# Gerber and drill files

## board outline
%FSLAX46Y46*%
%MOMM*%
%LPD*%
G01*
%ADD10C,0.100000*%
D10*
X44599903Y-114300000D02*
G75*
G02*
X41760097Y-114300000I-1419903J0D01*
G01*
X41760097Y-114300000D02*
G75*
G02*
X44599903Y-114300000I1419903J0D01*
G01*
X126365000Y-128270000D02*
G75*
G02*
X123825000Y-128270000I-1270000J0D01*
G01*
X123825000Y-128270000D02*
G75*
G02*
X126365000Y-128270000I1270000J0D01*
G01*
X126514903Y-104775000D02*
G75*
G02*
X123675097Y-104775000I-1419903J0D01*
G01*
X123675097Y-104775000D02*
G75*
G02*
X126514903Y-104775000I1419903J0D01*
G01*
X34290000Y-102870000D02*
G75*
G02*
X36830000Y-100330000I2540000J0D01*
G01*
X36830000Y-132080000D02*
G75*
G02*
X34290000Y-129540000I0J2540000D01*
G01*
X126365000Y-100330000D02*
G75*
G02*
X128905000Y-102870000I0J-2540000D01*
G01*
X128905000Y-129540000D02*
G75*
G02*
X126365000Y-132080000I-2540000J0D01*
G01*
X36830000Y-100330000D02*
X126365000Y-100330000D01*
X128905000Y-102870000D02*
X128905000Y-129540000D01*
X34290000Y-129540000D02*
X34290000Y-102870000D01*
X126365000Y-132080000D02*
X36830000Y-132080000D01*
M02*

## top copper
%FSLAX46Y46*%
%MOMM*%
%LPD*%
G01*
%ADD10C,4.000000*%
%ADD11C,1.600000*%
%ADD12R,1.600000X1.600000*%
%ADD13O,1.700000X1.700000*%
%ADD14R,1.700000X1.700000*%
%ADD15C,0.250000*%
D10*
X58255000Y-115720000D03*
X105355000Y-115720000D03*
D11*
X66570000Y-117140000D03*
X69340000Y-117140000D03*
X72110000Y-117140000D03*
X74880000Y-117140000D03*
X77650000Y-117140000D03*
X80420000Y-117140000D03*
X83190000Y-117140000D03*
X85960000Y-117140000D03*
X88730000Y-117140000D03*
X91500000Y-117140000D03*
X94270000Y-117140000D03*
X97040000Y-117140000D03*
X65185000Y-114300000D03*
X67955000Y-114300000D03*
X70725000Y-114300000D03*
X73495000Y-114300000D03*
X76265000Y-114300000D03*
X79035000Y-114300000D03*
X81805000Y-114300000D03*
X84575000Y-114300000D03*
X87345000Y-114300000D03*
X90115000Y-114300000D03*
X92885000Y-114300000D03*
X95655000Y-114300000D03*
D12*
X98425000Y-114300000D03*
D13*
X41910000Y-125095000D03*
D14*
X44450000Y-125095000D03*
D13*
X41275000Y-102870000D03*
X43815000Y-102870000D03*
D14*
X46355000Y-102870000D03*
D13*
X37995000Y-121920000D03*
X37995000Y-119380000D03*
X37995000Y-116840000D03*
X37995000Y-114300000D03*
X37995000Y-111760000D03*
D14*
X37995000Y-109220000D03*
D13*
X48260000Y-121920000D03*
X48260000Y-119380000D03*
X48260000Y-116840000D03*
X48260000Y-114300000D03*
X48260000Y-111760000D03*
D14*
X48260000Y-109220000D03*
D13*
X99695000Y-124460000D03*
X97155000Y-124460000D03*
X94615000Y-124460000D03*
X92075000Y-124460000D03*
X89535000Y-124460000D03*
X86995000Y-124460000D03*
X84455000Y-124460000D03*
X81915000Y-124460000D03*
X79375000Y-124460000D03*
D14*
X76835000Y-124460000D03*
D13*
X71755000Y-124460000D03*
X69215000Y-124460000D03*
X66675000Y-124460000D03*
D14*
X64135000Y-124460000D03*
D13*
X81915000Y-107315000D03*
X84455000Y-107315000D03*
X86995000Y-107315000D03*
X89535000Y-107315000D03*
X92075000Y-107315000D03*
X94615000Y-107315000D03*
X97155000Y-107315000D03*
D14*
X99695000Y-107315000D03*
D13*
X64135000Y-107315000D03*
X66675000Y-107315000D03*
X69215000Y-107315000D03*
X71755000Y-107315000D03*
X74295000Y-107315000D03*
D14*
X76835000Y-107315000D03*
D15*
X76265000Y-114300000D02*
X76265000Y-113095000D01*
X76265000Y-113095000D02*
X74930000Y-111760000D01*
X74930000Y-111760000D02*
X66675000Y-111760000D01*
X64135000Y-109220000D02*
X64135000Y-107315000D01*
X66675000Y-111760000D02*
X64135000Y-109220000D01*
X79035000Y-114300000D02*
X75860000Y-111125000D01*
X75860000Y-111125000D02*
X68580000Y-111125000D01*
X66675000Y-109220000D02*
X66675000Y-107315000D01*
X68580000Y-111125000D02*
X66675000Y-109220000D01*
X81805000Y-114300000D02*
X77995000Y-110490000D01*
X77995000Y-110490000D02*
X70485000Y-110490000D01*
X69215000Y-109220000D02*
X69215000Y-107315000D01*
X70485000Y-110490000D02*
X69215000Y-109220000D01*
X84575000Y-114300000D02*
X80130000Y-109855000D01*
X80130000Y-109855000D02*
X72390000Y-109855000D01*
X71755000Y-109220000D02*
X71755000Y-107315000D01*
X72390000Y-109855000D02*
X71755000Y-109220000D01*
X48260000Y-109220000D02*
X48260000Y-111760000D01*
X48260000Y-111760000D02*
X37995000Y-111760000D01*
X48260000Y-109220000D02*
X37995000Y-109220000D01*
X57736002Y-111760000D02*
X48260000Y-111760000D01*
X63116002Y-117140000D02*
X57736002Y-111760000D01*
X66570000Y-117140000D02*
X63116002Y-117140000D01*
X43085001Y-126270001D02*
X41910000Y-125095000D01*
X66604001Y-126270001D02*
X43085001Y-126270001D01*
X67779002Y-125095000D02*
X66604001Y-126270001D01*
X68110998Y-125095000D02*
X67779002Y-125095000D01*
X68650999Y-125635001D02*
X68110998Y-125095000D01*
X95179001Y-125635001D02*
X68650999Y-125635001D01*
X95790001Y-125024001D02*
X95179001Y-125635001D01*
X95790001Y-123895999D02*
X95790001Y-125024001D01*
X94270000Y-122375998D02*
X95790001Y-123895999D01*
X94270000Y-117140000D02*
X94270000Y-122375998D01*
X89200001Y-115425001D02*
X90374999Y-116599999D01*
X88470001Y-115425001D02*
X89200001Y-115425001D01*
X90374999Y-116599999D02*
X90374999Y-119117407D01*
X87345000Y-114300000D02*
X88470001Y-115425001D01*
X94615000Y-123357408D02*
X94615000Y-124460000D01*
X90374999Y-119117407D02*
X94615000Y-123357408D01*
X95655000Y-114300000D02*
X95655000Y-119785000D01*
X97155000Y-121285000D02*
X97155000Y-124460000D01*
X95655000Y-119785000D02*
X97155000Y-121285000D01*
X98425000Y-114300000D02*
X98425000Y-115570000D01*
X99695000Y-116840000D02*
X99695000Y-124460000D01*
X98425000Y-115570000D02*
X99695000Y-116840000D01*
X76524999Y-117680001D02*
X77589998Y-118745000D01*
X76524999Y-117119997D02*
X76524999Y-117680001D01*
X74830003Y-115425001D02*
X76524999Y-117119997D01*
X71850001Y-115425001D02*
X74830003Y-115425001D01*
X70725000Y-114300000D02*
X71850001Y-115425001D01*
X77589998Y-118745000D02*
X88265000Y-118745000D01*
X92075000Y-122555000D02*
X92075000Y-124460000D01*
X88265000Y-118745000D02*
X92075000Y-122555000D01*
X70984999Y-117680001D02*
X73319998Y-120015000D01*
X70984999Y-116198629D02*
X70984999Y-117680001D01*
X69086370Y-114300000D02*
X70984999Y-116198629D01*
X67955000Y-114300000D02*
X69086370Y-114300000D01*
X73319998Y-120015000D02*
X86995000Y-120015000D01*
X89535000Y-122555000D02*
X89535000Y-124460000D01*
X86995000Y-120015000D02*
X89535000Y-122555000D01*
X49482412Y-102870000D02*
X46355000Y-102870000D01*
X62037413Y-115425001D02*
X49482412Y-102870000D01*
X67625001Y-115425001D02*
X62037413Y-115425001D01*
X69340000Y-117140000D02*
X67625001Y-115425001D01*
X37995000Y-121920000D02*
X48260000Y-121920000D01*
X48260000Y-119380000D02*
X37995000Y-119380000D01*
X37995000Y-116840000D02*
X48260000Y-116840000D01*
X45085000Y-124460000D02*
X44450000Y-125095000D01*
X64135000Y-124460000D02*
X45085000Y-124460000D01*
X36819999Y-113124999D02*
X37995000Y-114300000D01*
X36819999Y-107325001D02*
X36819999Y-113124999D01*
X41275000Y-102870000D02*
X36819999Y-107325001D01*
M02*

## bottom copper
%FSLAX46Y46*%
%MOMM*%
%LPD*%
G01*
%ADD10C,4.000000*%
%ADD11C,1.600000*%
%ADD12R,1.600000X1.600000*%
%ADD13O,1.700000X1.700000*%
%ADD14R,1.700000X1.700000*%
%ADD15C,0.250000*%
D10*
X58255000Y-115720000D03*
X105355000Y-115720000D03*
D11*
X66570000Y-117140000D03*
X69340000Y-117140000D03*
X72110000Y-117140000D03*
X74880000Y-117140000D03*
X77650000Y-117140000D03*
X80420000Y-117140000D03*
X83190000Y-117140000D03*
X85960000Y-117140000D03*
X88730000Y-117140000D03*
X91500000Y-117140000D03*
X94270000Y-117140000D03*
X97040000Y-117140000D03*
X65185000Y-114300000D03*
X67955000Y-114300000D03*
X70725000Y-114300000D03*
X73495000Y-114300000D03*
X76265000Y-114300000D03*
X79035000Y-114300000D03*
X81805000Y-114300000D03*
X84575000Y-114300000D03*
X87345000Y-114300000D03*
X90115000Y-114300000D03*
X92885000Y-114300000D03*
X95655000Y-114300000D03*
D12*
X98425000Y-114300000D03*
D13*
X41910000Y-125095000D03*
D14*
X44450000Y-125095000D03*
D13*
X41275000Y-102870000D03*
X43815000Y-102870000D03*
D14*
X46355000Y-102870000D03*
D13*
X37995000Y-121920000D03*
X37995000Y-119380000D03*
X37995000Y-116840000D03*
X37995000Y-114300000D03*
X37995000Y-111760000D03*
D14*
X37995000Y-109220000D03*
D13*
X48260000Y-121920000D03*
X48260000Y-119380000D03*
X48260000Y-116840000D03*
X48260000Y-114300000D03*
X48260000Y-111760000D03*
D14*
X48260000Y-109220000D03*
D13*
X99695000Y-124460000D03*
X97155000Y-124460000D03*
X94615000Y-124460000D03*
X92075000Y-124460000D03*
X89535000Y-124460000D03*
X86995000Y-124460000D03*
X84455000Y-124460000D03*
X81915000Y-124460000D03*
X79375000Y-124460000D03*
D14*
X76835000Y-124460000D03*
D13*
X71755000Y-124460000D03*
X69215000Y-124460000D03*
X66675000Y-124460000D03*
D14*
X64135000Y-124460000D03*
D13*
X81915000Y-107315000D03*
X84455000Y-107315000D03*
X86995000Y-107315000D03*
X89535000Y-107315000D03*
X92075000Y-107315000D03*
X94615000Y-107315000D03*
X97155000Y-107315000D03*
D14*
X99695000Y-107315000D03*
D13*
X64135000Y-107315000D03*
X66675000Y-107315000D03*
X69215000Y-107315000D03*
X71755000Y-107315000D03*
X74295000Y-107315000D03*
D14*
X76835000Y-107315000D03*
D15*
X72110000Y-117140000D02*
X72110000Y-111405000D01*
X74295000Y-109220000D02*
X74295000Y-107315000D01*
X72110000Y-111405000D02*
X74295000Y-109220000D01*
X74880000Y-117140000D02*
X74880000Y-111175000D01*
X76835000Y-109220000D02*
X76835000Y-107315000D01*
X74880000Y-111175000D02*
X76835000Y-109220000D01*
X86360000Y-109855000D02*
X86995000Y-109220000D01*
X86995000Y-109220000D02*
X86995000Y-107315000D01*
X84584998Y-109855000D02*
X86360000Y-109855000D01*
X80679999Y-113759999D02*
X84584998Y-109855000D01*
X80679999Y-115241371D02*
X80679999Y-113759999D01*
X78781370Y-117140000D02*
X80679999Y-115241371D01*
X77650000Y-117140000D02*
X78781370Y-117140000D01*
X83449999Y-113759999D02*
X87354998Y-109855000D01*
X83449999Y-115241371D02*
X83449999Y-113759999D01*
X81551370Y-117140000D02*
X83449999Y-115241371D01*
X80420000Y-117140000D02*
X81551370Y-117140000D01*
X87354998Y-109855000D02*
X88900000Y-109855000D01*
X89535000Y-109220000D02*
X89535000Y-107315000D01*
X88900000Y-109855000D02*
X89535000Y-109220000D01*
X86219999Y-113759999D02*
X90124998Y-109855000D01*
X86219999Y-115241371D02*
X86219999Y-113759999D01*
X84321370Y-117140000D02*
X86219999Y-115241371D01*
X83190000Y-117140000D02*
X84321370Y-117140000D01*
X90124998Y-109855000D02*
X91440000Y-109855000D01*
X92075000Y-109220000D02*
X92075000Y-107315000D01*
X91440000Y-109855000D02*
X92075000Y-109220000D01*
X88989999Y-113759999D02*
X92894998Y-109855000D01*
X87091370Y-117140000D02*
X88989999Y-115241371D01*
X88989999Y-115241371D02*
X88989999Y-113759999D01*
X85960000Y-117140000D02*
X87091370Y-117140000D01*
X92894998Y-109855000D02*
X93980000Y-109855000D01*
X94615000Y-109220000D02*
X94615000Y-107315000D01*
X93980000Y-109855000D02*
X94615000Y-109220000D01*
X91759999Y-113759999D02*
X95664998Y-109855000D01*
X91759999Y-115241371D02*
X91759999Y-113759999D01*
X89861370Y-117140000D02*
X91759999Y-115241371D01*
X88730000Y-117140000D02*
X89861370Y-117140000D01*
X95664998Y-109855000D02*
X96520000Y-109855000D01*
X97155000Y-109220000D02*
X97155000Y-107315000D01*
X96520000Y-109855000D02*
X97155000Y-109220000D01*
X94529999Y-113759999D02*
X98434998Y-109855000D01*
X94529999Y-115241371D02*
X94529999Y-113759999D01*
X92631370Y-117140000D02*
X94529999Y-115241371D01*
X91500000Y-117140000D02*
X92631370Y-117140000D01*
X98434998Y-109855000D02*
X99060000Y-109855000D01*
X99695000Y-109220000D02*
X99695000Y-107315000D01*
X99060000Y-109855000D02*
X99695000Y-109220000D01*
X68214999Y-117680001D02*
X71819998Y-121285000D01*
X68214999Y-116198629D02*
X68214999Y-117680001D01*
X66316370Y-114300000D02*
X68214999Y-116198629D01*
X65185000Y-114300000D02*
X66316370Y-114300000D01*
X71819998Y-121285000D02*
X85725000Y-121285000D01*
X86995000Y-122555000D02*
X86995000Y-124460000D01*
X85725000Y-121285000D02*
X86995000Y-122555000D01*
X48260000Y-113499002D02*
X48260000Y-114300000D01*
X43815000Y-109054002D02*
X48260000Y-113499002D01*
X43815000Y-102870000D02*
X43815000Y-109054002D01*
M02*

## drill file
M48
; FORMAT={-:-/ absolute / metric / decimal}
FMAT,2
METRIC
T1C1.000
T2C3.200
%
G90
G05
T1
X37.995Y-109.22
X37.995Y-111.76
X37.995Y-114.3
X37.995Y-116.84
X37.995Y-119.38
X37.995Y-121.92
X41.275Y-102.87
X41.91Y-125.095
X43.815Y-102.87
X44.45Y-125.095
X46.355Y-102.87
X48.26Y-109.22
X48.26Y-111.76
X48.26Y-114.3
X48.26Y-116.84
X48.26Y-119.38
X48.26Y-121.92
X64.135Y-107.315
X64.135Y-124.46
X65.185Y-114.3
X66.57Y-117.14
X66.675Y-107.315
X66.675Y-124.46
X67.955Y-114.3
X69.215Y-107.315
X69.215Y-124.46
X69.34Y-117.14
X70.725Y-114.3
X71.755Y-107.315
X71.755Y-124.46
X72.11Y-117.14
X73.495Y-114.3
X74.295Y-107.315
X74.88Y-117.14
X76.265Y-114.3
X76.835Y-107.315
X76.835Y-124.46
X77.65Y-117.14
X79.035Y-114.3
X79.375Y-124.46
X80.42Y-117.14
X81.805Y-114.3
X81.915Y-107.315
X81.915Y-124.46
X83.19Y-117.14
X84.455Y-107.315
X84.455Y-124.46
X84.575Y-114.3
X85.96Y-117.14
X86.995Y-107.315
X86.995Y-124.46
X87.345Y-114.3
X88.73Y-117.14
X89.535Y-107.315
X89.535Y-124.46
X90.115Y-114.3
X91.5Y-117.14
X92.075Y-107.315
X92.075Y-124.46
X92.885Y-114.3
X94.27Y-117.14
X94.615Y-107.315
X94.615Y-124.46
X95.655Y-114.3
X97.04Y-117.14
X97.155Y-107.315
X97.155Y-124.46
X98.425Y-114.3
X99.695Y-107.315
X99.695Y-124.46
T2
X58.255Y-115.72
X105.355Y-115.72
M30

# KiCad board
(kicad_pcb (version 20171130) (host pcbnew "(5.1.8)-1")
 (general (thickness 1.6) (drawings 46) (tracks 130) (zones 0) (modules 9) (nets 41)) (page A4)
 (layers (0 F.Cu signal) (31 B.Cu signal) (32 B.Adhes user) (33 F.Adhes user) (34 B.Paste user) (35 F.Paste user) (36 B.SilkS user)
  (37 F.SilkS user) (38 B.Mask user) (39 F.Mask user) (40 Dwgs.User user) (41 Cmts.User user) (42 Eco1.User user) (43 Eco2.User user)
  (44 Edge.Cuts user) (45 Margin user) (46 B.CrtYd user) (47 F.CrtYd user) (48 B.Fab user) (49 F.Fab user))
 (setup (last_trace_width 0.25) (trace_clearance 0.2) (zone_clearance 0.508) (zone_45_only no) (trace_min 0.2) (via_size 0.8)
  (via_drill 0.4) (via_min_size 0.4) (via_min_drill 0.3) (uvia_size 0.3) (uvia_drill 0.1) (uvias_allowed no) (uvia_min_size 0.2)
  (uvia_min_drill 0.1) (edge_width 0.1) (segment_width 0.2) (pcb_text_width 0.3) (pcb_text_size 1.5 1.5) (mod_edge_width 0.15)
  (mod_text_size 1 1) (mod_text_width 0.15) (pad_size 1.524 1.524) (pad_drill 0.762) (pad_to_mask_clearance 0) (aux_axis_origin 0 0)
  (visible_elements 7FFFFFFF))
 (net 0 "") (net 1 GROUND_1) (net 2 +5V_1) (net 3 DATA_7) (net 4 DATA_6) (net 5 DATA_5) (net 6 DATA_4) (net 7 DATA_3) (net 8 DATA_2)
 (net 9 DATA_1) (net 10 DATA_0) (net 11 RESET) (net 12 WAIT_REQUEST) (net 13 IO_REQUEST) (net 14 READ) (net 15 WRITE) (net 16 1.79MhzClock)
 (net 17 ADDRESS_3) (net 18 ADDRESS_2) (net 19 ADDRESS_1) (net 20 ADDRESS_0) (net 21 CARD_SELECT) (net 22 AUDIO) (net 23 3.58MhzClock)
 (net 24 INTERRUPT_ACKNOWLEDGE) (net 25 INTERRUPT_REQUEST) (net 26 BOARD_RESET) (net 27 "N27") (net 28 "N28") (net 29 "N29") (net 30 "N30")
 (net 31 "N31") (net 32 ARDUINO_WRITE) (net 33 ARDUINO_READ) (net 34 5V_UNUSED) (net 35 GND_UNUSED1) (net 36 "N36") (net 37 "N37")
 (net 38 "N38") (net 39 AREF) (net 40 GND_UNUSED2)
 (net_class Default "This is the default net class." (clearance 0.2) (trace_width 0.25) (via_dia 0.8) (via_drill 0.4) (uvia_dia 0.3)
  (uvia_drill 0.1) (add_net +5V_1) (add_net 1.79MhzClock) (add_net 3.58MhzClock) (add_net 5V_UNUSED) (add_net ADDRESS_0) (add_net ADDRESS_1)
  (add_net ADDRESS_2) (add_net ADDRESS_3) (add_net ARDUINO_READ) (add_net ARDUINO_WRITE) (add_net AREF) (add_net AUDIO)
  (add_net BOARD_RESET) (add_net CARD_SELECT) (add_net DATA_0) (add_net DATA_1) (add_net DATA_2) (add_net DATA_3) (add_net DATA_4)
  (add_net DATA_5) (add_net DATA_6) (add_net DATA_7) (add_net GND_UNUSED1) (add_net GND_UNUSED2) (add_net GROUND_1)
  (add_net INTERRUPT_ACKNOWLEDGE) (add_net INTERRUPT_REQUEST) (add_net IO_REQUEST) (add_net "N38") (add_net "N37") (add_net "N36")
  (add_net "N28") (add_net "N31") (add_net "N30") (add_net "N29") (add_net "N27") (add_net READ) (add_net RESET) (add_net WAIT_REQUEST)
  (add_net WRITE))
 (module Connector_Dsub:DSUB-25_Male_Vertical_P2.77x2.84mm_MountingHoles (layer B.Cu) (at 98.425 114.3 180)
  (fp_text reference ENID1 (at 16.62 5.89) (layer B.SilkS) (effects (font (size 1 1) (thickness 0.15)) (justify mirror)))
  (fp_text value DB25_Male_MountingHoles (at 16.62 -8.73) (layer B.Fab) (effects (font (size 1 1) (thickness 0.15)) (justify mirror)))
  (pad 0 thru_hole circle (at 40.17 -1.42 180) (size 4 4) (drill 3.2) (layers *.Cu *.Mask))
  (pad 0 thru_hole circle (at -6.93 -1.42 180) (size 4 4) (drill 3.2) (layers *.Cu *.Mask))
  (pad 25 thru_hole circle (at 31.855 -2.84 180) (size 1.6 1.6) (drill 1) (layers *.Cu *.Mask) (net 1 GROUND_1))
  (pad 24 thru_hole circle (at 29.085 -2.84 180) (size 1.6 1.6) (drill 1) (layers *.Cu *.Mask) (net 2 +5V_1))
  (pad 23 thru_hole circle (at 26.315 -2.84 180) (size 1.6 1.6) (drill 1) (layers *.Cu *.Mask) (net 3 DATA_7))
  (pad 22 thru_hole circle (at 23.545 -2.84 180) (size 1.6 1.6) (drill 1) (layers *.Cu *.Mask) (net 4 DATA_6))
  (pad 21 thru_hole circle (at 20.775 -2.84 180) (size 1.6 1.6) (drill 1) (layers *.Cu *.Mask) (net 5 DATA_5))
  (pad 20 thru_hole circle (at 18.005 -2.84 180) (size 1.6 1.6) (drill 1) (layers *.Cu *.Mask) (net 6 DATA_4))
  (pad 19 thru_hole circle (at 15.235 -2.84 180) (size 1.6 1.6) (drill 1) (layers *.Cu *.Mask) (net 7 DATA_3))
  (pad 18 thru_hole circle (at 12.465 -2.84 180) (size 1.6 1.6) (drill 1) (layers *.Cu *.Mask) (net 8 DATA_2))
  (pad 17 thru_hole circle (at 9.695 -2.84 180) (size 1.6 1.6) (drill 1) (layers *.Cu *.Mask) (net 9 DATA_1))
  (pad 16 thru_hole circle (at 6.925 -2.84 180) (size 1.6 1.6) (drill 1) (layers *.Cu *.Mask) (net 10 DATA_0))
  (pad 15 thru_hole circle (at 4.155 -2.84 180) (size 1.6 1.6) (drill 1) (layers *.Cu *.Mask) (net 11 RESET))
  (pad 14 thru_hole circle (at 1.385 -2.84 180) (size 1.6 1.6) (drill 1) (layers *.Cu *.Mask) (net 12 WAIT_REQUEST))
  (pad 13 thru_hole circle (at 33.24 0 180) (size 1.6 1.6) (drill 1) (layers *.Cu *.Mask) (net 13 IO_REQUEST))
  (pad 12 thru_hole circle (at 30.47 0 180) (size 1.6 1.6) (drill 1) (layers *.Cu *.Mask) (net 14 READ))
  (pad 11 thru_hole circle (at 27.7 0 180) (size 1.6 1.6) (drill 1) (layers *.Cu *.Mask) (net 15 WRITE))
  (pad 10 thru_hole circle (at 24.93 0 180) (size 1.6 1.6) (drill 1) (layers *.Cu *.Mask) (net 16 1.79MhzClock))
  (pad 9 thru_hole circle (at 22.16 0 180) (size 1.6 1.6) (drill 1) (layers *.Cu *.Mask) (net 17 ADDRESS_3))
  (pad 8 thru_hole circle (at 19.39 0 180) (size 1.6 1.6) (drill 1) (layers *.Cu *.Mask) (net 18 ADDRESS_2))
  (pad 7 thru_hole circle (at 16.62 0 180) (size 1.6 1.6) (drill 1) (layers *.Cu *.Mask) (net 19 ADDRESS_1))
  (pad 6 thru_hole circle (at 13.85 0 180) (size 1.6 1.6) (drill 1) (layers *.Cu *.Mask) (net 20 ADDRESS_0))
  (pad 5 thru_hole circle (at 11.08 0 180) (size 1.6 1.6) (drill 1) (layers *.Cu *.Mask) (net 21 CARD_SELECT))
  (pad 4 thru_hole circle (at 8.31 0 180) (size 1.6 1.6) (drill 1) (layers *.Cu *.Mask) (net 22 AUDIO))
  (pad 3 thru_hole circle (at 5.54 0 180) (size 1.6 1.6) (drill 1) (layers *.Cu *.Mask) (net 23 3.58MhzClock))
  (pad 2 thru_hole circle (at 2.77 0 180) (size 1.6 1.6) (drill 1) (layers *.Cu *.Mask) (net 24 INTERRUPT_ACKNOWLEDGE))
  (pad 1 thru_hole rect (at 0 0 180) (size 1.6 1.6) (drill 1) (layers *.Cu *.Mask) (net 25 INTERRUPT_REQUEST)))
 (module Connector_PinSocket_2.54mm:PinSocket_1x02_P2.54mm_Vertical (layer F.Cu) (at 44.45 125.095 270)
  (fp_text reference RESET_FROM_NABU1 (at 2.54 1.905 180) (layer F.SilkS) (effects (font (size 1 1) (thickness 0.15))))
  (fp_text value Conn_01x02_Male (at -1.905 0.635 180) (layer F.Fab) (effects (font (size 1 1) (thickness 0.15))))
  (pad 2 thru_hole oval (at 0 2.54 270) (size 1.7 1.7) (drill 1) (layers *.Cu *.Mask) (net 11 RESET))
  (pad 1 thru_hole rect (at 0 0 270) (size 1.7 1.7) (drill 1) (layers *.Cu *.Mask) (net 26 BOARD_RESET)))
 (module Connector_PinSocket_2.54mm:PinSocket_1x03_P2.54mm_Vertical (layer F.Cu) (at 46.355 102.87 270)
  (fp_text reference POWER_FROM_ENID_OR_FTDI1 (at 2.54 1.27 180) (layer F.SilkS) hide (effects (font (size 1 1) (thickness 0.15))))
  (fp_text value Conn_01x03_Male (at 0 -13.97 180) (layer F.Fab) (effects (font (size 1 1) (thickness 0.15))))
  (pad 3 thru_hole oval (at 0 5.08 270) (size 1.7 1.7) (drill 1) (layers *.Cu *.Mask) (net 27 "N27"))
  (pad 2 thru_hole oval (at 0 2.54 270) (size 1.7 1.7) (drill 1) (layers *.Cu *.Mask) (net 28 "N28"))
  (pad 1 thru_hole rect (at 0 0 270) (size 1.7 1.7) (drill 1) (layers *.Cu *.Mask) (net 2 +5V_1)))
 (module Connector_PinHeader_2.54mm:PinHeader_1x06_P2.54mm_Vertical (layer F.Cu) (at 37.995 109.22)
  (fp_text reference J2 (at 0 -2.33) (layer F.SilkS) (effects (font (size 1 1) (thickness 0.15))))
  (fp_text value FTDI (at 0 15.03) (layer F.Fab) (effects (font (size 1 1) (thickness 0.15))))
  (pad 6 thru_hole oval (at 0 12.7) (size 1.7 1.7) (drill 1) (layers *.Cu *.Mask) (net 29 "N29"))
  (pad 5 thru_hole oval (at 0 10.16) (size 1.7 1.7) (drill 1) (layers *.Cu *.Mask) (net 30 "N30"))
  (pad 4 thru_hole oval (at 0 7.62) (size 1.7 1.7) (drill 1) (layers *.Cu *.Mask) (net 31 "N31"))
  (pad 3 thru_hole oval (at 0 5.08) (size 1.7 1.7) (drill 1) (layers *.Cu *.Mask) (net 27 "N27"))
  (pad 2 thru_hole oval (at 0 2.54) (size 1.7 1.7) (drill 1) (layers *.Cu *.Mask) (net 1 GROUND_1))
  (pad 1 thru_hole rect (at 0 0) (size 1.7 1.7) (drill 1) (layers *.Cu *.Mask) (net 1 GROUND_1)))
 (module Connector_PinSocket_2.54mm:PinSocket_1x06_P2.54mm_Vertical (layer F.Cu) (at 48.26 109.22)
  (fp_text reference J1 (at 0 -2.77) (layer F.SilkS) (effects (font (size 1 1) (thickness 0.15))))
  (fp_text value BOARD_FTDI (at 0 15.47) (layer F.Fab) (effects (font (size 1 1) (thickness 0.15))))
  (pad 6 thru_hole oval (at 0 12.7) (size 1.7 1.7) (drill 1) (layers *.Cu *.Mask) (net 29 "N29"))
  (pad 5 thru_hole oval (at 0 10.16) (size 1.7 1.7) (drill 1) (layers *.Cu *.Mask) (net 30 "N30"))
  (pad 4 thru_hole oval (at 0 7.62) (size 1.7 1.7) (drill 1) (layers *.Cu *.Mask) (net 31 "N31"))
  (pad 3 thru_hole oval (at 0 5.08) (size 1.7 1.7) (drill 1) (layers *.Cu *.Mask) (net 28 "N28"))
  (pad 2 thru_hole oval (at 0 2.54) (size 1.7 1.7) (drill 1) (layers *.Cu *.Mask) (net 1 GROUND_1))
  (pad 1 thru_hole rect (at 0 0) (size 1.7 1.7) (drill 1) (layers *.Cu *.Mask) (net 1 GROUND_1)))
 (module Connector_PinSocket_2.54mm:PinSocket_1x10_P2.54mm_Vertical (layer F.Cu) (at 76.835 124.46 90)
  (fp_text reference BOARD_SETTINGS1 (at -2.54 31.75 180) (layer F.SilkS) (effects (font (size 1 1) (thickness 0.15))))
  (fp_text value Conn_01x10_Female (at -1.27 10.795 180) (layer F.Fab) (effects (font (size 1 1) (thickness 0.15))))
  (pad 10 thru_hole oval (at 0 22.86 90) (size 1.7 1.7) (drill 1) (layers *.Cu *.Mask) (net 25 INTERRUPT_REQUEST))
  (pad 9 thru_hole oval (at 0 20.32 90) (size 1.7 1.7) (drill 1) (layers *.Cu *.Mask) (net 24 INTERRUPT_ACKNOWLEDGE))
  (pad 8 thru_hole oval (at 0 17.78 90) (size 1.7 1.7) (drill 1) (layers *.Cu *.Mask) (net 21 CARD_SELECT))
  (pad 7 thru_hole oval (at 0 15.24 90) (size 1.7 1.7) (drill 1) (layers *.Cu *.Mask) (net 15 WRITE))
  (pad 6 thru_hole oval (at 0 12.7 90) (size 1.7 1.7) (drill 1) (layers *.Cu *.Mask) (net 14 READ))
  (pad 5 thru_hole oval (at 0 10.16 90) (size 1.7 1.7) (drill 1) (layers *.Cu *.Mask) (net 13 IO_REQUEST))
  (pad 4 thru_hole oval (at 0 7.62 90) (size 1.7 1.7) (drill 1) (layers *.Cu *.Mask) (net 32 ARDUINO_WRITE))
  (pad 3 thru_hole oval (at 0 5.08 90) (size 1.7 1.7) (drill 1) (layers *.Cu *.Mask) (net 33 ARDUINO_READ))
  (pad 2 thru_hole oval (at 0 2.54 90) (size 1.7 1.7) (drill 1) (layers *.Cu *.Mask) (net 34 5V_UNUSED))
  (pad 1 thru_hole rect (at 0 0 90) (size 1.7 1.7) (drill 1) (layers *.Cu *.Mask) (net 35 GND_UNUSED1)))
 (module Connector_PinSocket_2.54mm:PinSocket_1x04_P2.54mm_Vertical (layer F.Cu) (at 64.135 124.46 90)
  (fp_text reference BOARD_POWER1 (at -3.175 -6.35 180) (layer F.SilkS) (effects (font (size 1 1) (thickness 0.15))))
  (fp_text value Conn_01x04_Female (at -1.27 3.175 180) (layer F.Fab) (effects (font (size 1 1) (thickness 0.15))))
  (pad 4 thru_hole oval (at 0 7.62 90) (size 1.7 1.7) (drill 1) (layers *.Cu *.Mask) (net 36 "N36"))
  (pad 3 thru_hole oval (at 0 5.08 90) (size 1.7 1.7) (drill 1) (layers *.Cu *.Mask) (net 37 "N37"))
  (pad 2 thru_hole oval (at 0 2.54 90) (size 1.7 1.7) (drill 1) (layers *.Cu *.Mask) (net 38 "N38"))
  (pad 1 thru_hole rect (at 0 0 90) (size 1.7 1.7) (drill 1) (layers *.Cu *.Mask) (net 26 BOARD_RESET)))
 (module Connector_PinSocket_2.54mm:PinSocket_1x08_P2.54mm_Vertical (layer F.Cu) (at 99.695 107.315 270)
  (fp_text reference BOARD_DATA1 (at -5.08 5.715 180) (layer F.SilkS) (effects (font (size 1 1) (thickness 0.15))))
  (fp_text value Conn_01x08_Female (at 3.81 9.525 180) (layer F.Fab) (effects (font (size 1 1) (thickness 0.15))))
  (pad 8 thru_hole oval (at 0 17.78 270) (size 1.7 1.7) (drill 1) (layers *.Cu *.Mask) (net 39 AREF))
  (pad 7 thru_hole oval (at 0 15.24 270) (size 1.7 1.7) (drill 1) (layers *.Cu *.Mask) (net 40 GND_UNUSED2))
  (pad 6 thru_hole oval (at 0 12.7 270) (size 1.7 1.7) (drill 1) (layers *.Cu *.Mask) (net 5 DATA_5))
  (pad 5 thru_hole oval (at 0 10.16 270) (size 1.7 1.7) (drill 1) (layers *.Cu *.Mask) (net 6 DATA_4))
  (pad 4 thru_hole oval (at 0 7.62 270) (size 1.7 1.7) (drill 1) (layers *.Cu *.Mask) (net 7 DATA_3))
  (pad 3 thru_hole oval (at 0 5.08 270) (size 1.7 1.7) (drill 1) (layers *.Cu *.Mask) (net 8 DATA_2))
  (pad 2 thru_hole oval (at 0 2.54 270) (size 1.7 1.7) (drill 1) (layers *.Cu *.Mask) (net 9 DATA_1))
  (pad 1 thru_hole rect (at 0 0 270) (size 1.7 1.7) (drill 1) (layers *.Cu *.Mask) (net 10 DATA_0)))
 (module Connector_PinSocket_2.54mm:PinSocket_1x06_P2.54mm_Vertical (layer F.Cu) (at 76.835 107.315 270)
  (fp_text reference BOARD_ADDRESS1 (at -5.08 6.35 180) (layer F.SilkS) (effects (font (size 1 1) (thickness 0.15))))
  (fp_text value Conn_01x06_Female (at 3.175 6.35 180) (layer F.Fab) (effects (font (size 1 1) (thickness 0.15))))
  (pad 6 thru_hole oval (at 0 12.7 270) (size 1.7 1.7) (drill 1) (layers *.Cu *.Mask) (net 17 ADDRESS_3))
  (pad 5 thru_hole oval (at 0 10.16 270) (size 1.7 1.7) (drill 1) (layers *.Cu *.Mask) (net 18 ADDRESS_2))
  (pad 4 thru_hole oval (at 0 7.62 270) (size 1.7 1.7) (drill 1) (layers *.Cu *.Mask) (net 19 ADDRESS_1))
  (pad 3 thru_hole oval (at 0 5.08 270) (size 1.7 1.7) (drill 1) (layers *.Cu *.Mask) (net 20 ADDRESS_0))
  (pad 2 thru_hole oval (at 0 2.54 270) (size 1.7 1.7) (drill 1) (layers *.Cu *.Mask) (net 3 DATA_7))
  (pad 1 thru_hole rect (at 0 0 270) (size 1.7 1.7) (drill 1) (layers *.Cu *.Mask) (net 4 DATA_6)))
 (gr_circle (center 43.18 114.3) (end 44.45 113.665) (layer Edge.Cuts) (width 0.1))
 (gr_circle (center 125.095 128.27) (end 125.095 129.54) (layer Edge.Cuts) (width 0.1))
 (gr_circle (center 125.095 104.775) (end 126.365 104.14) (layer Edge.Cuts) (width 0.1))
 (gr_arc (start 36.83 102.87) (end 36.83 100.33) (angle -90) (layer Edge.Cuts) (width 0.1))
 (gr_arc (start 36.83 129.54) (end 34.29 129.54) (angle -90) (layer Edge.Cuts) (width 0.1))
 (gr_arc (start 126.365 102.87) (end 128.905 102.87) (angle -90) (layer Edge.Cuts) (width 0.1))
 (gr_arc (start 126.365 129.54) (end 126.365 132.08) (angle -90) (layer Edge.Cuts) (width 0.1))
 (gr_line (start 36.83 100.33) (end 126.365 100.33) (layer Edge.Cuts) (width 0.1))
 (gr_line (start 128.905 102.87) (end 128.905 129.54) (layer Edge.Cuts) (width 0.1))
 (gr_line (start 34.29 129.54) (end 34.29 102.87) (layer Edge.Cuts) (width 0.1))
 (gr_line (start 126.365 132.08) (end 36.83 132.08) (layer Edge.Cuts) (width 0.1))
 (segment (start 76.265 114.3) (end 76.265 113.095) (width 0.25) (layer F.Cu) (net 17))
 (segment (start 76.265 113.095) (end 74.93 111.76) (width 0.25) (layer F.Cu) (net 17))
 (segment (start 74.93 111.76) (end 66.675 111.76) (width 0.25) (layer F.Cu) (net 17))
 (segment (start 64.135 109.22) (end 64.135 107.315) (width 0.25) (layer F.Cu) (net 17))
 (segment (start 66.675 111.76) (end 64.135 109.22) (width 0.25) (layer F.Cu) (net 17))
 (segment (start 79.035 114.3) (end 75.86 111.125) (width 0.25) (layer F.Cu) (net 18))
 (segment (start 75.86 111.125) (end 68.58 111.125) (width 0.25) (layer F.Cu) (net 18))
 (segment (start 66.675 109.22) (end 66.675 107.315) (width 0.25) (layer F.Cu) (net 18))
 (segment (start 68.58 111.125) (end 66.675 109.22) (width 0.25) (layer F.Cu) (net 18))
 (segment (start 81.805 114.3) (end 77.995 110.49) (width 0.25) (layer F.Cu) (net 19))
 (segment (start 77.995 110.49) (end 70.485 110.49) (width 0.25) (layer F.Cu) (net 19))
 (segment (start 69.215 109.22) (end 69.215 107.315) (width 0.25) (layer F.Cu) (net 19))
 (segment (start 70.485 110.49) (end 69.215 109.22) (width 0.25) (layer F.Cu) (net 19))
 (segment (start 84.575 114.3) (end 80.13 109.855) (width 0.25) (layer F.Cu) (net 20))
 (segment (start 80.13 109.855) (end 72.39 109.855) (width 0.25) (layer F.Cu) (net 20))
 (segment (start 71.755 109.22) (end 71.755 107.315) (width 0.25) (layer F.Cu) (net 20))
 (segment (start 72.39 109.855) (end 71.755 109.22) (width 0.25) (layer F.Cu) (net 20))
 (segment (start 72.11 117.14) (end 72.11 111.405) (width 0.25) (layer B.Cu) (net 3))
 (segment (start 74.295 109.22) (end 74.295 107.315) (width 0.25) (layer B.Cu) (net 3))
 (segment (start 72.11 111.405) (end 74.295 109.22) (width 0.25) (layer B.Cu) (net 3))
 (segment (start 74.88 117.14) (end 74.88 111.175) (width 0.25) (layer B.Cu) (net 4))
 (segment (start 76.835 109.22) (end 76.835 107.315) (width 0.25) (layer B.Cu) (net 4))
 (segment (start 74.88 111.175) (end 76.835 109.22) (width 0.25) (layer B.Cu) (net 4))
 (segment (start 86.36 109.855) (end 86.995 109.22) (width 0.25) (layer B.Cu) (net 5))
 (segment (start 86.995 109.22) (end 86.995 107.315) (width 0.25) (layer B.Cu) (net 5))
 (segment (start 84.584998 109.855) (end 86.36 109.855) (width 0.25) (layer B.Cu) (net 5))
 (segment (start 80.679999 113.759999) (end 84.584998 109.855) (width 0.25) (layer B.Cu) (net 5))
 (segment (start 80.679999 115.241371) (end 80.679999 113.759999) (width 0.25) (layer B.Cu) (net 5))
 (segment (start 78.78137 117.14) (end 80.679999 115.241371) (width 0.25) (layer B.Cu) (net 5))
 (segment (start 77.65 117.14) (end 78.78137 117.14) (width 0.25) (layer B.Cu) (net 5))
 (segment (start 83.449999 113.759999) (end 87.354998 109.855) (width 0.25) (layer B.Cu) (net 6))
 (segment (start 83.449999 115.241371) (end 83.449999 113.759999) (width 0.25) (layer B.Cu) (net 6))
 (segment (start 81.55137 117.14) (end 83.449999 115.241371) (width 0.25) (layer B.Cu) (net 6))
 (segment (start 80.42 117.14) (end 81.55137 117.14) (width 0.25) (layer B.Cu) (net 6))
 (segment (start 87.354998 109.855) (end 88.9 109.855) (width 0.25) (layer B.Cu) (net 6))
 (segment (start 89.535 109.22) (end 89.535 107.315) (width 0.25) (layer B.Cu) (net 6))
 (segment (start 88.9 109.855) (end 89.535 109.22) (width 0.25) (layer B.Cu) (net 6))
 (segment (start 86.219999 113.759999) (end 90.124998 109.855) (width 0.25) (layer B.Cu) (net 7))
 (segment (start 86.219999 115.241371) (end 86.219999 113.759999) (width 0.25) (layer B.Cu) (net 7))
 (segment (start 84.32137 117.14) (end 86.219999 115.241371) (width 0.25) (layer B.Cu) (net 7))
 (segment (start 83.19 117.14) (end 84.32137 117.14) (width 0.25) (layer B.Cu) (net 7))
 (segment (start 90.124998 109.855) (end 91.44 109.855) (width 0.25) (layer B.Cu) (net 7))
 (segment (start 92.075 109.22) (end 92.075 107.315) (width 0.25) (layer B.Cu) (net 7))
 (segment (start 91.44 109.855) (end 92.075 109.22) (width 0.25) (layer B.Cu) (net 7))
 (segment (start 88.989999 113.759999) (end 92.894998 109.855) (width 0.25) (layer B.Cu) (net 8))
 (segment (start 87.09137 117.14) (end 88.989999 115.241371) (width 0.25) (layer B.Cu) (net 8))
 (segment (start 88.989999 115.241371) (end 88.989999 113.759999) (width 0.25) (layer B.Cu) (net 8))
 (segment (start 85.96 117.14) (end 87.09137 117.14) (width 0.25) (layer B.Cu) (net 8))
 (segment (start 92.894998 109.855) (end 93.98 109.855) (width 0.25) (layer B.Cu) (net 8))
 (segment (start 94.615 109.22) (end 94.615 107.315) (width 0.25) (layer B.Cu) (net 8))
 (segment (start 93.98 109.855) (end 94.615 109.22) (width 0.25) (layer B.Cu) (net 8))
 (segment (start 91.759999 113.759999) (end 95.664998 109.855) (width 0.25) (layer B.Cu) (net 9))
 (segment (start 91.759999 115.241371) (end 91.759999 113.759999) (width 0.25) (layer B.Cu) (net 9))
 (segment (start 89.86137 117.14) (end 91.759999 115.241371) (width 0.25) (layer B.Cu) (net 9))
 (segment (start 88.73 117.14) (end 89.86137 117.14) (width 0.25) (layer B.Cu) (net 9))
 (segment (start 95.664998 109.855) (end 96.52 109.855) (width 0.25) (layer B.Cu) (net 9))
 (segment (start 97.155 109.22) (end 97.155 107.315) (width 0.25) (layer B.Cu) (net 9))
 (segment (start 96.52 109.855) (end 97.155 109.22) (width 0.25) (layer B.Cu) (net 9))
 (segment (start 94.529999 113.759999) (end 98.434998 109.855) (width 0.25) (layer B.Cu) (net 10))
 (segment (start 94.529999 115.241371) (end 94.529999 113.759999) (width 0.25) (layer B.Cu) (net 10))
 (segment (start 92.63137 117.14) (end 94.529999 115.241371) (width 0.25) (layer B.Cu) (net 10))
 (segment (start 91.5 117.14) (end 92.63137 117.14) (width 0.25) (layer B.Cu) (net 10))
 (segment (start 98.434998 109.855) (end 99.06 109.855) (width 0.25) (layer B.Cu) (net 10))
 (segment (start 99.695 109.22) (end 99.695 107.315) (width 0.25) (layer B.Cu) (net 10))
 (segment (start 99.06 109.855) (end 99.695 109.22) (width 0.25) (layer B.Cu) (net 10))
 (segment (start 48.26 109.22) (end 48.26 111.76) (width 0.25) (layer F.Cu) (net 1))
 (segment (start 48.26 111.76) (end 37.995 111.76) (width 0.25) (layer F.Cu) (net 1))
 (segment (start 48.26 109.22) (end 37.995 109.22) (width 0.25) (layer F.Cu) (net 1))
 (segment (start 57.736002 111.76) (end 48.26 111.76) (width 0.25) (layer F.Cu) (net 1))
 (segment (start 63.116002 117.14) (end 57.736002 111.76) (width 0.25) (layer F.Cu) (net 1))
 (segment (start 66.57 117.14) (end 63.116002 117.14) (width 0.25) (layer F.Cu) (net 1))
 (segment (start 43.085001 126.270001) (end 41.91 125.095) (width 0.25) (layer F.Cu) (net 11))
 (segment (start 66.604001 126.270001) (end 43.085001 126.270001) (width 0.25) (layer F.Cu) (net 11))
 (segment (start 67.779002 125.095) (end 66.604001 126.270001) (width 0.25) (layer F.Cu) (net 11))
 (segment (start 68.110998 125.095) (end 67.779002 125.095) (width 0.25) (layer F.Cu) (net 11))
 (segment (start 68.650999 125.635001) (end 68.110998 125.095) (width 0.25) (layer F.Cu) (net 11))
 (segment (start 95.179001 125.635001) (end 68.650999 125.635001) (width 0.25) (layer F.Cu) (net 11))
 (segment (start 95.790001 125.024001) (end 95.179001 125.635001) (width 0.25) (layer F.Cu) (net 11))
 (segment (start 95.790001 123.895999) (end 95.790001 125.024001) (width 0.25) (layer F.Cu) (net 11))
 (segment (start 94.27 122.375998) (end 95.790001 123.895999) (width 0.25) (layer F.Cu) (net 11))
 (segment (start 94.27 117.14) (end 94.27 122.375998) (width 0.25) (layer F.Cu) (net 11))
 (segment (start 89.200001 115.425001) (end 90.374999 116.599999) (width 0.25) (layer F.Cu) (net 21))
 (segment (start 88.470001 115.425001) (end 89.200001 115.425001) (width 0.25) (layer F.Cu) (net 21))
 (segment (start 90.374999 116.599999) (end 90.374999 119.117407) (width 0.25) (layer F.Cu) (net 21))
 (segment (start 87.345 114.3) (end 88.470001 115.425001) (width 0.25) (layer F.Cu) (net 21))
 (segment (start 94.615 123.357408) (end 94.615 124.46) (width 0.25) (layer F.Cu) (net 21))
 (segment (start 90.374999 119.117407) (end 94.615 123.357408) (width 0.25) (layer F.Cu) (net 21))
 (segment (start 95.655 114.3) (end 95.655 119.785) (width 0.25) (layer F.Cu) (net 24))
 (segment (start 97.155 121.285) (end 97.155 124.46) (width 0.25) (layer F.Cu) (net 24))
 (segment (start 95.655 119.785) (end 97.155 121.285) (width 0.25) (layer F.Cu) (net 24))
 (segment (start 98.425 114.3) (end 98.425 115.57) (width 0.25) (layer F.Cu) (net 25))
 (segment (start 99.695 116.84) (end 99.695 124.46) (width 0.25) (layer F.Cu) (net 25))
 (segment (start 98.425 115.57) (end 99.695 116.84) (width 0.25) (layer F.Cu) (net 25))
 (segment (start 76.524999 117.680001) (end 77.589998 118.745) (width 0.25) (layer F.Cu) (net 15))
 (segment (start 76.524999 117.119997) (end 76.524999 117.680001) (width 0.25) (layer F.Cu) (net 15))
 (segment (start 74.830003 115.425001) (end 76.524999 117.119997) (width 0.25) (layer F.Cu) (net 15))
 (segment (start 71.850001 115.425001) (end 74.830003 115.425001) (width 0.25) (layer F.Cu) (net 15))
 (segment (start 70.725 114.3) (end 71.850001 115.425001) (width 0.25) (layer F.Cu) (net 15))
 (segment (start 77.589998 118.745) (end 88.265 118.745) (width 0.25) (layer F.Cu) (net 15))
 (segment (start 92.075 122.555) (end 92.075 124.46) (width 0.25) (layer F.Cu) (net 15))
 (segment (start 88.265 118.745) (end 92.075 122.555) (width 0.25) (layer F.Cu) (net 15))
 (segment (start 70.984999 117.680001) (end 73.319998 120.015) (width 0.25) (layer F.Cu) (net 14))
 (segment (start 70.984999 116.198629) (end 70.984999 117.680001) (width 0.25) (layer F.Cu) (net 14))
 (segment (start 69.08637 114.3) (end 70.984999 116.198629) (width 0.25) (layer F.Cu) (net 14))
 (segment (start 67.955 114.3) (end 69.08637 114.3) (width 0.25) (layer F.Cu) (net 14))
 (segment (start 73.319998 120.015) (end 86.995 120.015) (width 0.25) (layer F.Cu) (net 14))
 (segment (start 89.535 122.555) (end 89.535 124.46) (width 0.25) (layer F.Cu) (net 14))
 (segment (start 86.995 120.015) (end 89.535 122.555) (width 0.25) (layer F.Cu) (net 14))
 (segment (start 68.214999 117.680001) (end 71.819998 121.285) (width 0.25) (layer B.Cu) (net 13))
 (segment (start 68.214999 116.198629) (end 68.214999 117.680001) (width 0.25) (layer B.Cu) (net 13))
 (segment (start 66.31637 114.3) (end 68.214999 116.198629) (width 0.25) (layer B.Cu) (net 13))
 (segment (start 65.185 114.3) (end 66.31637 114.3) (width 0.25) (layer B.Cu) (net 13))
 (segment (start 71.819998 121.285) (end 85.725 121.285) (width 0.25) (layer B.Cu) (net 13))
 (segment (start 86.995 122.555) (end 86.995 124.46) (width 0.25) (layer B.Cu) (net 13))
 (segment (start 85.725 121.285) (end 86.995 122.555) (width 0.25) (layer B.Cu) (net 13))
 (segment (start 49.482412 102.87) (end 46.355 102.87) (width 0.25) (layer F.Cu) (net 2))
 (segment (start 62.037413 115.425001) (end 49.482412 102.87) (width 0.25) (layer F.Cu) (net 2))
 (segment (start 67.625001 115.425001) (end 62.037413 115.425001) (width 0.25) (layer F.Cu) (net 2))
 (segment (start 69.34 117.14) (end 67.625001 115.425001) (width 0.25) (layer F.Cu) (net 2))
 (segment (start 37.995 121.92) (end 48.26 121.92) (width 0.25) (layer F.Cu) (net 29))
 (segment (start 48.26 119.38) (end 37.995 119.38) (width 0.25) (layer F.Cu) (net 30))
 (segment (start 37.995 116.84) (end 48.26 116.84) (width 0.25) (layer F.Cu) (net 31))
 (segment (start 48.26 113.499002) (end 48.26 114.3) (width 0.25) (layer B.Cu) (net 28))
 (segment (start 43.815 109.054002) (end 48.26 113.499002) (width 0.25) (layer B.Cu) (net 28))
 (segment (start 43.815 102.87) (end 43.815 109.054002) (width 0.25) (layer B.Cu) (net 28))
 (segment (start 45.085 124.46) (end 44.45 125.095) (width 0.25) (layer F.Cu) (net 26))
 (segment (start 64.135 124.46) (end 45.085 124.46) (width 0.25) (layer F.Cu) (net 26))
 (segment (start 36.819999 113.124999) (end 37.995 114.3) (width 0.25) (layer F.Cu) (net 27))
 (segment (start 36.819999 107.325001) (end 36.819999 113.124999) (width 0.25) (layer F.Cu) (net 27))
 (segment (start 41.275 102.87) (end 36.819999 107.325001) (width 0.25) (layer F.Cu) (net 27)))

